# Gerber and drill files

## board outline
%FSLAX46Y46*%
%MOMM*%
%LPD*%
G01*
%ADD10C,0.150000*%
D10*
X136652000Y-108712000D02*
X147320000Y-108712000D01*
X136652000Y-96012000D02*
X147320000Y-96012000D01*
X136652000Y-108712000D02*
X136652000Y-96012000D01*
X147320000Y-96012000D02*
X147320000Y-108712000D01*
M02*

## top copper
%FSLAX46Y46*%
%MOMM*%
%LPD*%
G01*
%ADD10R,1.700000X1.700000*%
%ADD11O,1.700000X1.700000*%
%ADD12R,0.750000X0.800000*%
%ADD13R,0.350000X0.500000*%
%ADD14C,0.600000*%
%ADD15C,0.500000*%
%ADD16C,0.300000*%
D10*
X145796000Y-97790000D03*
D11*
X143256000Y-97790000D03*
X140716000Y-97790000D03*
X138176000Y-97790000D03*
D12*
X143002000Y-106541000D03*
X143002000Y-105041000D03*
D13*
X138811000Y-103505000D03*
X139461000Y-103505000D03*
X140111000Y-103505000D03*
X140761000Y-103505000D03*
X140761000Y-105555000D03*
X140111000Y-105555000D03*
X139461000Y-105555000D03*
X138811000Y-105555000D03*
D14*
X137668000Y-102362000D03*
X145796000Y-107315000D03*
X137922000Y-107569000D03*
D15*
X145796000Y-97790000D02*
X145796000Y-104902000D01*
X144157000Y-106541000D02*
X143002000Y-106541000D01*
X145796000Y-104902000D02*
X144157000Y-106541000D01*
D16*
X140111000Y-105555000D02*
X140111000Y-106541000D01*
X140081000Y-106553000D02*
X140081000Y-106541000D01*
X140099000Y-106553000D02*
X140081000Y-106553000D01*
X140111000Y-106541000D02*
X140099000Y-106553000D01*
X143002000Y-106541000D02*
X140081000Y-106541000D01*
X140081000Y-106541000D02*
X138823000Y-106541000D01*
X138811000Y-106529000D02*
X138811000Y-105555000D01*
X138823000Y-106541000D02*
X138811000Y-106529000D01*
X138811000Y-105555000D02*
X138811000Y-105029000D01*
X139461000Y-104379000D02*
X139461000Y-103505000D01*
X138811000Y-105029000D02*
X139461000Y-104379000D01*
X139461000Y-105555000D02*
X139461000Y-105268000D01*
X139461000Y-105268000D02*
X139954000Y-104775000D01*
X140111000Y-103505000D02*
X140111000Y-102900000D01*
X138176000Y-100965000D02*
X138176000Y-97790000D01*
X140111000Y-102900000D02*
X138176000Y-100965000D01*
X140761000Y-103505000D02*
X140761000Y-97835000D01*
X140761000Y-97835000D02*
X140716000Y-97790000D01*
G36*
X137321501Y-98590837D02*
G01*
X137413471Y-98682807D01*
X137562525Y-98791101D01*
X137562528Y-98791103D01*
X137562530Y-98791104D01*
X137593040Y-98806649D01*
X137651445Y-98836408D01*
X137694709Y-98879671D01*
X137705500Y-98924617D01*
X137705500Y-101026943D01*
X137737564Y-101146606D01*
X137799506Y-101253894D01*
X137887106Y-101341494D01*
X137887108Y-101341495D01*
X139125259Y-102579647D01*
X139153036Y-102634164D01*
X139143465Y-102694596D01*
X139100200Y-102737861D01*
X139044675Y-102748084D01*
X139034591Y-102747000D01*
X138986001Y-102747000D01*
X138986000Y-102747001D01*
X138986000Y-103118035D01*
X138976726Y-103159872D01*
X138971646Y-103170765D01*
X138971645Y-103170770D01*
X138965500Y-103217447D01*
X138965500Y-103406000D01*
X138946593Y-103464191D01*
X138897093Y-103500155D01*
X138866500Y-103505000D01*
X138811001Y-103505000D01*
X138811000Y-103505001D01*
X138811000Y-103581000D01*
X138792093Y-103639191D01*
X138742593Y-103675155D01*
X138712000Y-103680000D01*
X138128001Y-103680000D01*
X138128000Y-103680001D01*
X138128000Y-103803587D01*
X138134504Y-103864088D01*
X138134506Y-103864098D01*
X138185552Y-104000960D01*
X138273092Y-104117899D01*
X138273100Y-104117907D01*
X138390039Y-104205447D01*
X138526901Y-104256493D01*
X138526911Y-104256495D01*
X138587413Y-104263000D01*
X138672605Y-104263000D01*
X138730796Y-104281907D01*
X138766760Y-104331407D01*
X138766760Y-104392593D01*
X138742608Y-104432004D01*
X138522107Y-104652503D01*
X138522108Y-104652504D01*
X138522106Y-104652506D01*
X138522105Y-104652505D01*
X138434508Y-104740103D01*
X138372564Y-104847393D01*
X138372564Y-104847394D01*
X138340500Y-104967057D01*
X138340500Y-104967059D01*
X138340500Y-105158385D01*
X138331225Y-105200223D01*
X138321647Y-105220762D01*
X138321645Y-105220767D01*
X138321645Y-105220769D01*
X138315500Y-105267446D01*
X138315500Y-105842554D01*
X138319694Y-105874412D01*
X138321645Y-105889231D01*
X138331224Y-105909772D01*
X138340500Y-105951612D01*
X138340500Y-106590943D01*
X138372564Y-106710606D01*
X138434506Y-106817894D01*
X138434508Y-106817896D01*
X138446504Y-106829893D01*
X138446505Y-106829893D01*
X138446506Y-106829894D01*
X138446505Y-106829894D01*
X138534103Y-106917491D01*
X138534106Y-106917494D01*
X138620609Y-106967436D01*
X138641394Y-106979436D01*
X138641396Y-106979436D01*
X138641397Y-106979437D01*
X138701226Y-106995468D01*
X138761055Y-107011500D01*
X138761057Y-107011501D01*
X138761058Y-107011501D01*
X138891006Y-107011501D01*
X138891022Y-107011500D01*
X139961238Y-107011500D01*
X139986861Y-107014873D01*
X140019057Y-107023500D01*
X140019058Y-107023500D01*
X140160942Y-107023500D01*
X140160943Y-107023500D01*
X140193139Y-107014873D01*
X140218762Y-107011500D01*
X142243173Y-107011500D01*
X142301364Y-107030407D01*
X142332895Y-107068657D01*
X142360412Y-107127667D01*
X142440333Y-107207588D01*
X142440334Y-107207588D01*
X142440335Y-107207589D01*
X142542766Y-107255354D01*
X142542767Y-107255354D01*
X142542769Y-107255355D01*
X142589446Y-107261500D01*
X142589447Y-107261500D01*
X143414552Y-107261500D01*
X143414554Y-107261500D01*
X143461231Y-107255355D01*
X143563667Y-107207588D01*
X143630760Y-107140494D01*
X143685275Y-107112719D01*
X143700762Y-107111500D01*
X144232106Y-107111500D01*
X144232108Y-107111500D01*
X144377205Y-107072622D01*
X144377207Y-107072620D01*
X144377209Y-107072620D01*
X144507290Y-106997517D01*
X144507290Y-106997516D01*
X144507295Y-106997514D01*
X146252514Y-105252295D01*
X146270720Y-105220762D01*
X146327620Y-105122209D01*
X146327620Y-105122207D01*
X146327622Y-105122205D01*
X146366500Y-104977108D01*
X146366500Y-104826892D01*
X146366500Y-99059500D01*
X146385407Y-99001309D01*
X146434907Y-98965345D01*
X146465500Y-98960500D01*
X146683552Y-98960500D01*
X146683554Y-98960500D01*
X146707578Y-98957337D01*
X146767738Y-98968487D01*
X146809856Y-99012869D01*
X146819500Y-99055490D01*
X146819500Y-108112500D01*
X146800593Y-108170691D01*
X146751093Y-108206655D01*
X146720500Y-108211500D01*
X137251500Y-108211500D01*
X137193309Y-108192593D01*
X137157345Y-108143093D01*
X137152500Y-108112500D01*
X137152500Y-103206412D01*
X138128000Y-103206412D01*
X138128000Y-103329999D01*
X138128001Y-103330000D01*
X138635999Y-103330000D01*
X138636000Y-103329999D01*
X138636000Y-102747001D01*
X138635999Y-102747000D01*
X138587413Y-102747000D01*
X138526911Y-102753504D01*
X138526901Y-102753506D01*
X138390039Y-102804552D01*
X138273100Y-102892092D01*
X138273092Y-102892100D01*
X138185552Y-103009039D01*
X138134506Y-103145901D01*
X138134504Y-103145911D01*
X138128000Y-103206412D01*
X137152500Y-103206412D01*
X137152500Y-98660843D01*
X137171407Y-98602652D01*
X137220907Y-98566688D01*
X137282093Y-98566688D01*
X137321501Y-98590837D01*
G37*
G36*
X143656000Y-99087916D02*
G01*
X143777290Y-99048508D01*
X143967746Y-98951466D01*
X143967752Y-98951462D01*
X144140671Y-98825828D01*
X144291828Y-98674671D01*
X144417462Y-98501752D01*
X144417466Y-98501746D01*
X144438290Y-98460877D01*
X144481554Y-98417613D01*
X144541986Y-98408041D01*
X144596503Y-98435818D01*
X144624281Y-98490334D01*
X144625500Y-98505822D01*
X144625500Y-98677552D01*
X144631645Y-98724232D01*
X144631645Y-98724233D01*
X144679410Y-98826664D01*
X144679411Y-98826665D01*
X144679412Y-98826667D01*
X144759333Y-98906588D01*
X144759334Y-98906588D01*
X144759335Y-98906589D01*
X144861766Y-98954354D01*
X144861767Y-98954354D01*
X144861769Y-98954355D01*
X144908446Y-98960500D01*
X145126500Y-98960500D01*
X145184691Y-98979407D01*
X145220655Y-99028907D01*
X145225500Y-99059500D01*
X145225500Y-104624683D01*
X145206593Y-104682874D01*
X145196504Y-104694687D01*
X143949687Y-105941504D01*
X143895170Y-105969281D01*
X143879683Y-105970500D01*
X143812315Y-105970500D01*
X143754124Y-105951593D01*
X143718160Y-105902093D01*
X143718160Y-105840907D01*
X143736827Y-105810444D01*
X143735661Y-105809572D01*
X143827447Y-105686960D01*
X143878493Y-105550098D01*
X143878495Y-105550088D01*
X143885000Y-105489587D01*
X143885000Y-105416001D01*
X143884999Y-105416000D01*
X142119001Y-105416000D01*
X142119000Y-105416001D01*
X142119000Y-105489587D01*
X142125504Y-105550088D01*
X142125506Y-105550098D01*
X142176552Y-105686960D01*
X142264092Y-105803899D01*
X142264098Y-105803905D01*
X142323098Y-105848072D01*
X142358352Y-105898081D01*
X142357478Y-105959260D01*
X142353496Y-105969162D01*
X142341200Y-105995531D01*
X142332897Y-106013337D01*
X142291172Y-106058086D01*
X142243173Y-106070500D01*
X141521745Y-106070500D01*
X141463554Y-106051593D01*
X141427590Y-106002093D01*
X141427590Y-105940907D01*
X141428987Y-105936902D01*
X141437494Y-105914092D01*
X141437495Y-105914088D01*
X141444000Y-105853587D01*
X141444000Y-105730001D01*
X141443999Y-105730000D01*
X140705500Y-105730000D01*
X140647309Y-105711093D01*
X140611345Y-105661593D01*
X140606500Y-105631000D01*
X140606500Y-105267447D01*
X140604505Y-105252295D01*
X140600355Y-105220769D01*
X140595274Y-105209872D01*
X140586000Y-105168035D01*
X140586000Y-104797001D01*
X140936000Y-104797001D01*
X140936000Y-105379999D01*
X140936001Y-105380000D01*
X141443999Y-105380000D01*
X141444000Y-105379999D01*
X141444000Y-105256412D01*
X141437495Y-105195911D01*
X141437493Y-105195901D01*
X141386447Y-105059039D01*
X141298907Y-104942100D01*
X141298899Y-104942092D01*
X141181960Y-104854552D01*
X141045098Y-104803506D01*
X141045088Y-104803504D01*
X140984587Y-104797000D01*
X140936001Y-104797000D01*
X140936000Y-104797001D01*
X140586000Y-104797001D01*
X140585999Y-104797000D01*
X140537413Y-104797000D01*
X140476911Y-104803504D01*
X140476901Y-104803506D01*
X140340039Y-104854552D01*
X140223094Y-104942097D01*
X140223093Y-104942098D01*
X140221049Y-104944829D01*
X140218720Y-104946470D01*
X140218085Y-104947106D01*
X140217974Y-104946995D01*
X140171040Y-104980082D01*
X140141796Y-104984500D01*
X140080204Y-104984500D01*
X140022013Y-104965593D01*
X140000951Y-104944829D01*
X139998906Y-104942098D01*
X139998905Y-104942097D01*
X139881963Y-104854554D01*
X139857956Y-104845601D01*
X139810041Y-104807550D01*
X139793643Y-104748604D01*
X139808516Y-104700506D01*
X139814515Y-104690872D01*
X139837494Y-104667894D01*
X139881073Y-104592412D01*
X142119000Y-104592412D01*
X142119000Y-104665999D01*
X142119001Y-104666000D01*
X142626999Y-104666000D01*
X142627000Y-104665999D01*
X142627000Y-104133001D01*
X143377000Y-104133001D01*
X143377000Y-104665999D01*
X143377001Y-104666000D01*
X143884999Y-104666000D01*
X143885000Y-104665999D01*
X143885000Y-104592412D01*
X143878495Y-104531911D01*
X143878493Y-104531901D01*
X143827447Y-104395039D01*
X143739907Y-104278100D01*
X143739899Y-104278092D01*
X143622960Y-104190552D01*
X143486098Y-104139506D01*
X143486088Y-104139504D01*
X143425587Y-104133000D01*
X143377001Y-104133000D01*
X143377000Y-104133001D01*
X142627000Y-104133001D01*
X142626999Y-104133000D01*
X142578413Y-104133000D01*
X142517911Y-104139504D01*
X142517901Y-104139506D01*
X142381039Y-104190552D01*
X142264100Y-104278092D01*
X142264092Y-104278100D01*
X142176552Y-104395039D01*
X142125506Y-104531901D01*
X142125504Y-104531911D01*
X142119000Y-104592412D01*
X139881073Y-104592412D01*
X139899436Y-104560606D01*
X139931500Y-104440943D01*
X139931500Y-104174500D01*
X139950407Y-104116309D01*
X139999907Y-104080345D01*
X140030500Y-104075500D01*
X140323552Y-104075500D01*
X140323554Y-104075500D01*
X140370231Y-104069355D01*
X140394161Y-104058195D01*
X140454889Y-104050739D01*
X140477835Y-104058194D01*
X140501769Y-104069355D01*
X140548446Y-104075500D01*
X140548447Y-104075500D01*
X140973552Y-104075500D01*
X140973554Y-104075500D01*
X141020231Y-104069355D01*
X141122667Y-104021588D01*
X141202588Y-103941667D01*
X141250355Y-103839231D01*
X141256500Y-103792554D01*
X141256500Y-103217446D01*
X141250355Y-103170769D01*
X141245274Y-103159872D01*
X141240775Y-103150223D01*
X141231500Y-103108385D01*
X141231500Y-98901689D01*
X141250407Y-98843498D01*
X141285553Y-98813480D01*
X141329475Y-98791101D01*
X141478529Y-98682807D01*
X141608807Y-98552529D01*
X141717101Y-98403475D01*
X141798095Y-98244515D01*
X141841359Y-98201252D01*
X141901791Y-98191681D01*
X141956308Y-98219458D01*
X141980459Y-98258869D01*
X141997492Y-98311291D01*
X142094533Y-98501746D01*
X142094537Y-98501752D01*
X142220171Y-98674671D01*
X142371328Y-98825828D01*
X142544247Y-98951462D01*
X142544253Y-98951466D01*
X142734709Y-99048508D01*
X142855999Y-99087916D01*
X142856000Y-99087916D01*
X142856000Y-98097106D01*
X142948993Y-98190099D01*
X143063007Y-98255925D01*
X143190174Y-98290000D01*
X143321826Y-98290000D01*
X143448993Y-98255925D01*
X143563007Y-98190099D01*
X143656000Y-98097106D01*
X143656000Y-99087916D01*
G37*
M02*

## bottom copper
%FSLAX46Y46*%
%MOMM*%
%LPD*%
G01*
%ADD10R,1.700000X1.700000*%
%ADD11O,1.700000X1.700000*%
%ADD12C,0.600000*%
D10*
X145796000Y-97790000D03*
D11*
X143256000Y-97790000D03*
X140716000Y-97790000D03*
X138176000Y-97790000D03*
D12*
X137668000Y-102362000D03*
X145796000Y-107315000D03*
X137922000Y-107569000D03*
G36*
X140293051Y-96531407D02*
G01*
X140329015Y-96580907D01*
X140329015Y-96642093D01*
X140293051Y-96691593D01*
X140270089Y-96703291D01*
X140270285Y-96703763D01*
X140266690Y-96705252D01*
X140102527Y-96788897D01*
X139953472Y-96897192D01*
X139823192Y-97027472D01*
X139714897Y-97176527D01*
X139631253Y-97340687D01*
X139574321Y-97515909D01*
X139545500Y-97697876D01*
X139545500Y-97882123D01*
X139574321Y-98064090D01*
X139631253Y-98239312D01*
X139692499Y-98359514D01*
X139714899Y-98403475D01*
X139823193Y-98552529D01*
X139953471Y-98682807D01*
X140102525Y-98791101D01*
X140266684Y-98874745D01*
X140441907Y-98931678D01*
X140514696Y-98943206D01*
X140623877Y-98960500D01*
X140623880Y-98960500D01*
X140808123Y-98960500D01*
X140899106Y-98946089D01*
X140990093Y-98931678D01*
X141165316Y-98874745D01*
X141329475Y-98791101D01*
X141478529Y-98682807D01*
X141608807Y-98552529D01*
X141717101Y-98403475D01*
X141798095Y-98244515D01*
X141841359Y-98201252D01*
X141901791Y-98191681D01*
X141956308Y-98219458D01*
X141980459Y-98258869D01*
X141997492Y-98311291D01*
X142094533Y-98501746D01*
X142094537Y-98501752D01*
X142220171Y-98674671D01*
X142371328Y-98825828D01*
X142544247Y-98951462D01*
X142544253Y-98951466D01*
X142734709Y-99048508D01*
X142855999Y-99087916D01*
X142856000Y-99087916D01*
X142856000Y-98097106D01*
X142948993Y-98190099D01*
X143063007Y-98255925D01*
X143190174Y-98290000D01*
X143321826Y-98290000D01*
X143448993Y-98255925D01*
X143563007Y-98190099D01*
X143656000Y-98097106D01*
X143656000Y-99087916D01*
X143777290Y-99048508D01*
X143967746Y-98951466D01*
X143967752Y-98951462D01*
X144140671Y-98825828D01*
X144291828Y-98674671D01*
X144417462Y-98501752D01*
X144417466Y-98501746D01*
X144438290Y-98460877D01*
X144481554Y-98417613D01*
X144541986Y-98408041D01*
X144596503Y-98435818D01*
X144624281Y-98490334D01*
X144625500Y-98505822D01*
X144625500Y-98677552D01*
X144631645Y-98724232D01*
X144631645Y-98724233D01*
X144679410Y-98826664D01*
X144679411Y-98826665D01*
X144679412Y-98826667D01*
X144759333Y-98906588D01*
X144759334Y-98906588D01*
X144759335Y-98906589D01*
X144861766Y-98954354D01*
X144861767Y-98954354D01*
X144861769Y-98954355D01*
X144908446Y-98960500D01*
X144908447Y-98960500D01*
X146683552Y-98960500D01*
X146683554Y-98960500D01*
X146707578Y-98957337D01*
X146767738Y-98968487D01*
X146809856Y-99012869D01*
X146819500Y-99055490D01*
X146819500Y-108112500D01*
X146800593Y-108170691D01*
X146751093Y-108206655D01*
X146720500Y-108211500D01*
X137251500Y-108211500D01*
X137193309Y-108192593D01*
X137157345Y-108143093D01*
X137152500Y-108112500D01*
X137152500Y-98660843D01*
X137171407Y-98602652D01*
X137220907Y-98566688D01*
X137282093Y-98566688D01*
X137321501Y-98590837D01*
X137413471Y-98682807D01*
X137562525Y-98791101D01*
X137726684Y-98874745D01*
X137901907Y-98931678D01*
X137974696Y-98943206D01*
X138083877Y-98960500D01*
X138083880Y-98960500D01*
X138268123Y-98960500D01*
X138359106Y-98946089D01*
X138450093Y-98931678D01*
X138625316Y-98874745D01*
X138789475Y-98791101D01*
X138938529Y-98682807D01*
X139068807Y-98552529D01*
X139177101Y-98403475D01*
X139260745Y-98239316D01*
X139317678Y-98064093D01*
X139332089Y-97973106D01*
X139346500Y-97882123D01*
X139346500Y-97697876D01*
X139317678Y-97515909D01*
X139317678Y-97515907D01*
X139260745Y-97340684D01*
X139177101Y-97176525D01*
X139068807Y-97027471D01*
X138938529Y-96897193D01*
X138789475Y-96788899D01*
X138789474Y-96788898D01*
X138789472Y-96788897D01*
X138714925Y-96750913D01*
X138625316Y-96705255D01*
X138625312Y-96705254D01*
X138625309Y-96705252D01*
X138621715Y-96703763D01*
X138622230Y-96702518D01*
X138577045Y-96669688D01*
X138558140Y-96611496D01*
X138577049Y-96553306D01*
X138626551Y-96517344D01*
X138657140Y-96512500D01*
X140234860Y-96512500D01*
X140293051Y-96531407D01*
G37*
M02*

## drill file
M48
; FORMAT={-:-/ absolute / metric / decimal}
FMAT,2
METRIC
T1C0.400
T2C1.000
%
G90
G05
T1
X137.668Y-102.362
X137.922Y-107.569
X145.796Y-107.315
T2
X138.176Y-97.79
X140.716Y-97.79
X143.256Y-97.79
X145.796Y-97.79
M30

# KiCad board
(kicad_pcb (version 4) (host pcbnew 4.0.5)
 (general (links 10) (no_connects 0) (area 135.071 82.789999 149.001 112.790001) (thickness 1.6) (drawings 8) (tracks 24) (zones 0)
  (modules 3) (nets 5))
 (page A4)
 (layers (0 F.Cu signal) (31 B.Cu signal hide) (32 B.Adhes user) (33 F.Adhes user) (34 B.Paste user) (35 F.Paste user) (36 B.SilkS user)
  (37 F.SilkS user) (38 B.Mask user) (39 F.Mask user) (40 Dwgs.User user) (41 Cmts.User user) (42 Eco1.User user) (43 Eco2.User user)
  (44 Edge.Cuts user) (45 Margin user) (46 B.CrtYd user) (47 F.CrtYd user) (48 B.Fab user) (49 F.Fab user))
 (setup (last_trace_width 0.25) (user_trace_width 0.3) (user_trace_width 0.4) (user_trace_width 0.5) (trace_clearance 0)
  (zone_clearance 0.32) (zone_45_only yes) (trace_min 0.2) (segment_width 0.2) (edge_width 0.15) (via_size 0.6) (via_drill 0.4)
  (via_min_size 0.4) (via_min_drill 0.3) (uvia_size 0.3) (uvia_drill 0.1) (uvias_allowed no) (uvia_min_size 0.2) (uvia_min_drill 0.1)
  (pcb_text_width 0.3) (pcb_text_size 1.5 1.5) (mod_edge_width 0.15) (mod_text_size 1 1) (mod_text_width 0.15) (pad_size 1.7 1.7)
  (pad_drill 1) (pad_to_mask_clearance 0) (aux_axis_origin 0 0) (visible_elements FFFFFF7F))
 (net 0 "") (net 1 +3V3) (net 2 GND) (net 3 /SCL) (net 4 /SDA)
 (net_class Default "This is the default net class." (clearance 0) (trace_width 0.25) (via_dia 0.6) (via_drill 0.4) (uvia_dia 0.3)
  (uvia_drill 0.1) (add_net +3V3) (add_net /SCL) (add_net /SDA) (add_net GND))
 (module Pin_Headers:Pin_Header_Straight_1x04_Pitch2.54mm (layer F.Cu) (at 145.796 97.79 270)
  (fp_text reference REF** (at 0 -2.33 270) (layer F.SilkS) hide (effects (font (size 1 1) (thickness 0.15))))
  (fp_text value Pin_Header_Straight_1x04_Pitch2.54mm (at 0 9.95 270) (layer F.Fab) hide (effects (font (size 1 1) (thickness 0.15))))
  (pad 1 thru_hole rect (at 0 0 270) (size 1.7 1.7) (drill 1) (layers *.Cu *.Mask) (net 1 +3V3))
  (pad 2 thru_hole oval (at 0 2.54 270) (size 1.7 1.7) (drill 1) (layers *.Cu *.Mask) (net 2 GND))
  (pad 3 thru_hole oval (at 0 5.08 270) (size 1.7 1.7) (drill 1) (layers *.Cu *.Mask) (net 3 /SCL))
  (pad 4 thru_hole oval (at 0 7.62 270) (size 1.7 1.7) (drill 1) (layers *.Cu *.Mask) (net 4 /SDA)))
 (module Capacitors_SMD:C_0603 (layer F.Cu) (at 143.002 105.791 90)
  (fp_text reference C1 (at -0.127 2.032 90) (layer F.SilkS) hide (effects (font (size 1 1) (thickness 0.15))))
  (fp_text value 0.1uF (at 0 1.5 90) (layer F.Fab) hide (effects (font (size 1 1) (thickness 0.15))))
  (pad 1 smd rect (at -0.75 0 90) (size 0.8 0.75) (layers F.Cu F.Paste F.Mask) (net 1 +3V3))
  (pad 2 smd rect (at 0.75 0 90) (size 0.8 0.75) (layers F.Cu F.Paste F.Mask) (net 2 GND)))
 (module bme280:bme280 (layer F.Cu) (at 138.811 103.505 90)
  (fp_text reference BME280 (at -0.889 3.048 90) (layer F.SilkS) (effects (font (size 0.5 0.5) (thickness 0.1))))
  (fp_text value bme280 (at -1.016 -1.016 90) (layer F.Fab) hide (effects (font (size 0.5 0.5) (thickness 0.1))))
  (pad 1 smd rect (at 0 0 90) (size 0.5 0.35) (layers F.Cu F.Paste F.Mask) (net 2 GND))
  (pad 2 smd rect (at 0 0.65 90) (size 0.5 0.35) (layers F.Cu F.Paste F.Mask) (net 1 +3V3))
  (pad 3 smd rect (at 0 1.3 90) (size 0.5 0.35) (layers F.Cu F.Paste F.Mask) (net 4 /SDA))
  (pad 4 smd rect (at 0 1.95 90) (size 0.5 0.35) (layers F.Cu F.Paste F.Mask) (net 3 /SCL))
  (pad 5 smd rect (at -2.05 1.95 90) (size 0.5 0.35) (layers F.Cu F.Paste F.Mask) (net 2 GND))
  (pad 6 smd rect (at -2.05 1.3 90) (size 0.5 0.35) (layers F.Cu F.Paste F.Mask) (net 1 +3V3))
  (pad 7 smd rect (at -2.05 0.65 90) (size 0.5 0.35) (layers F.Cu F.Paste F.Mask) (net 2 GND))
  (pad 8 smd rect (at -2.05 0 90) (size 0.5 0.35) (layers F.Cu F.Paste F.Mask) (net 1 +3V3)))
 (gr_line (start 136.652 108.712) (end 147.32 108.712) (angle 90) (layer Edge.Cuts) (width 0.15))
 (gr_line (start 136.652 96.012) (end 147.32 96.012) (angle 90) (layer Edge.Cuts) (width 0.15))
 (gr_line (start 136.652 108.712) (end 136.652 96.012) (angle 90) (layer Edge.Cuts) (width 0.15))
 (gr_line (start 147.32 96.012) (end 147.32 108.712) (angle 90) (layer Edge.Cuts) (width 0.15))
 (segment (start 145.796 97.79) (end 145.796 104.902) (width 0.5) (layer F.Cu) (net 1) (status 10))
 (segment (start 144.157 106.541) (end 143.002 106.541) (width 0.5) (layer F.Cu) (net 1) (status 20))
 (segment (start 145.796 104.902) (end 144.157 106.541) (width 0.5) (layer F.Cu) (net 1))
 (segment (start 140.111 105.555) (end 140.111 106.541) (width 0.3) (layer F.Cu) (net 1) (status 10))
 (segment (start 140.081 106.553) (end 140.081 106.541) (width 0.3) (layer F.Cu) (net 1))
 (segment (start 140.099 106.553) (end 140.081 106.553) (width 0.3) (layer F.Cu) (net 1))
 (segment (start 140.111 106.541) (end 140.099 106.553) (width 0.3) (layer F.Cu) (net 1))
 (segment (start 143.002 106.541) (end 140.081 106.541) (width 0.3) (layer F.Cu) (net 1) (status 10))
 (segment (start 140.081 106.541) (end 138.823 106.541) (width 0.3) (layer F.Cu) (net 1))
 (segment (start 138.811 106.529) (end 138.811 105.555) (width 0.3) (layer F.Cu) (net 1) (status 20))
 (segment (start 138.823 106.541) (end 138.811 106.529) (width 0.3) (layer F.Cu) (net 1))
 (segment (start 138.811 105.555) (end 138.811 105.029) (width 0.3) (layer F.Cu) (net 1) (status 10))
 (segment (start 139.461 104.379) (end 139.461 103.505) (width 0.3) (layer F.Cu) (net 1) (status 20))
 (segment (start 138.811 105.029) (end 139.461 104.379) (width 0.3) (layer F.Cu) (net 1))
 (via (at 137.668 102.362) (size 0.6) (drill 0.4) (layers F.Cu B.Cu) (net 2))
 (via (at 145.796 107.315) (size 0.6) (drill 0.4) (layers F.Cu B.Cu) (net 2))
 (via (at 137.922 107.569) (size 0.6) (drill 0.4) (layers F.Cu B.Cu) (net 2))
 (segment (start 139.461 105.555) (end 139.461 105.268) (width 0.3) (layer F.Cu) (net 2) (status 10))
 (segment (start 139.461 105.268) (end 139.954 104.775) (width 0.3) (layer F.Cu) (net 2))
 (segment (start 140.111 103.505) (end 140.111 102.9) (width 0.3) (layer F.Cu) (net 4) (status 10))
 (segment (start 138.176 100.965) (end 138.176 97.79) (width 0.3) (layer F.Cu) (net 4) (status 20))
 (segment (start 140.111 102.9) (end 138.176 100.965) (width 0.3) (layer F.Cu) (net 4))
 (segment (start 140.761 103.505) (end 140.761 97.835) (width 0.3) (layer F.Cu) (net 3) (status 30))
 (segment (start 140.761 97.835) (end 140.716 97.79) (width 0.3) (layer F.Cu) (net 3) (status 30))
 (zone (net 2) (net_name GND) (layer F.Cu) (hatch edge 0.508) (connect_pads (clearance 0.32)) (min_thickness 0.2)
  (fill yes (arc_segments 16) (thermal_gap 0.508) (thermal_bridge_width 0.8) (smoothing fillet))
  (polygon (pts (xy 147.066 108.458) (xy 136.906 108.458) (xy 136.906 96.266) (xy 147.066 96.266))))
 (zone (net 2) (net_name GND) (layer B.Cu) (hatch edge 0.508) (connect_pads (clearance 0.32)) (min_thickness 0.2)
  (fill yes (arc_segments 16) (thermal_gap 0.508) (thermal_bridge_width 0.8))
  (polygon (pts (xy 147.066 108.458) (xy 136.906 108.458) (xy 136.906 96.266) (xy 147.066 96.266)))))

